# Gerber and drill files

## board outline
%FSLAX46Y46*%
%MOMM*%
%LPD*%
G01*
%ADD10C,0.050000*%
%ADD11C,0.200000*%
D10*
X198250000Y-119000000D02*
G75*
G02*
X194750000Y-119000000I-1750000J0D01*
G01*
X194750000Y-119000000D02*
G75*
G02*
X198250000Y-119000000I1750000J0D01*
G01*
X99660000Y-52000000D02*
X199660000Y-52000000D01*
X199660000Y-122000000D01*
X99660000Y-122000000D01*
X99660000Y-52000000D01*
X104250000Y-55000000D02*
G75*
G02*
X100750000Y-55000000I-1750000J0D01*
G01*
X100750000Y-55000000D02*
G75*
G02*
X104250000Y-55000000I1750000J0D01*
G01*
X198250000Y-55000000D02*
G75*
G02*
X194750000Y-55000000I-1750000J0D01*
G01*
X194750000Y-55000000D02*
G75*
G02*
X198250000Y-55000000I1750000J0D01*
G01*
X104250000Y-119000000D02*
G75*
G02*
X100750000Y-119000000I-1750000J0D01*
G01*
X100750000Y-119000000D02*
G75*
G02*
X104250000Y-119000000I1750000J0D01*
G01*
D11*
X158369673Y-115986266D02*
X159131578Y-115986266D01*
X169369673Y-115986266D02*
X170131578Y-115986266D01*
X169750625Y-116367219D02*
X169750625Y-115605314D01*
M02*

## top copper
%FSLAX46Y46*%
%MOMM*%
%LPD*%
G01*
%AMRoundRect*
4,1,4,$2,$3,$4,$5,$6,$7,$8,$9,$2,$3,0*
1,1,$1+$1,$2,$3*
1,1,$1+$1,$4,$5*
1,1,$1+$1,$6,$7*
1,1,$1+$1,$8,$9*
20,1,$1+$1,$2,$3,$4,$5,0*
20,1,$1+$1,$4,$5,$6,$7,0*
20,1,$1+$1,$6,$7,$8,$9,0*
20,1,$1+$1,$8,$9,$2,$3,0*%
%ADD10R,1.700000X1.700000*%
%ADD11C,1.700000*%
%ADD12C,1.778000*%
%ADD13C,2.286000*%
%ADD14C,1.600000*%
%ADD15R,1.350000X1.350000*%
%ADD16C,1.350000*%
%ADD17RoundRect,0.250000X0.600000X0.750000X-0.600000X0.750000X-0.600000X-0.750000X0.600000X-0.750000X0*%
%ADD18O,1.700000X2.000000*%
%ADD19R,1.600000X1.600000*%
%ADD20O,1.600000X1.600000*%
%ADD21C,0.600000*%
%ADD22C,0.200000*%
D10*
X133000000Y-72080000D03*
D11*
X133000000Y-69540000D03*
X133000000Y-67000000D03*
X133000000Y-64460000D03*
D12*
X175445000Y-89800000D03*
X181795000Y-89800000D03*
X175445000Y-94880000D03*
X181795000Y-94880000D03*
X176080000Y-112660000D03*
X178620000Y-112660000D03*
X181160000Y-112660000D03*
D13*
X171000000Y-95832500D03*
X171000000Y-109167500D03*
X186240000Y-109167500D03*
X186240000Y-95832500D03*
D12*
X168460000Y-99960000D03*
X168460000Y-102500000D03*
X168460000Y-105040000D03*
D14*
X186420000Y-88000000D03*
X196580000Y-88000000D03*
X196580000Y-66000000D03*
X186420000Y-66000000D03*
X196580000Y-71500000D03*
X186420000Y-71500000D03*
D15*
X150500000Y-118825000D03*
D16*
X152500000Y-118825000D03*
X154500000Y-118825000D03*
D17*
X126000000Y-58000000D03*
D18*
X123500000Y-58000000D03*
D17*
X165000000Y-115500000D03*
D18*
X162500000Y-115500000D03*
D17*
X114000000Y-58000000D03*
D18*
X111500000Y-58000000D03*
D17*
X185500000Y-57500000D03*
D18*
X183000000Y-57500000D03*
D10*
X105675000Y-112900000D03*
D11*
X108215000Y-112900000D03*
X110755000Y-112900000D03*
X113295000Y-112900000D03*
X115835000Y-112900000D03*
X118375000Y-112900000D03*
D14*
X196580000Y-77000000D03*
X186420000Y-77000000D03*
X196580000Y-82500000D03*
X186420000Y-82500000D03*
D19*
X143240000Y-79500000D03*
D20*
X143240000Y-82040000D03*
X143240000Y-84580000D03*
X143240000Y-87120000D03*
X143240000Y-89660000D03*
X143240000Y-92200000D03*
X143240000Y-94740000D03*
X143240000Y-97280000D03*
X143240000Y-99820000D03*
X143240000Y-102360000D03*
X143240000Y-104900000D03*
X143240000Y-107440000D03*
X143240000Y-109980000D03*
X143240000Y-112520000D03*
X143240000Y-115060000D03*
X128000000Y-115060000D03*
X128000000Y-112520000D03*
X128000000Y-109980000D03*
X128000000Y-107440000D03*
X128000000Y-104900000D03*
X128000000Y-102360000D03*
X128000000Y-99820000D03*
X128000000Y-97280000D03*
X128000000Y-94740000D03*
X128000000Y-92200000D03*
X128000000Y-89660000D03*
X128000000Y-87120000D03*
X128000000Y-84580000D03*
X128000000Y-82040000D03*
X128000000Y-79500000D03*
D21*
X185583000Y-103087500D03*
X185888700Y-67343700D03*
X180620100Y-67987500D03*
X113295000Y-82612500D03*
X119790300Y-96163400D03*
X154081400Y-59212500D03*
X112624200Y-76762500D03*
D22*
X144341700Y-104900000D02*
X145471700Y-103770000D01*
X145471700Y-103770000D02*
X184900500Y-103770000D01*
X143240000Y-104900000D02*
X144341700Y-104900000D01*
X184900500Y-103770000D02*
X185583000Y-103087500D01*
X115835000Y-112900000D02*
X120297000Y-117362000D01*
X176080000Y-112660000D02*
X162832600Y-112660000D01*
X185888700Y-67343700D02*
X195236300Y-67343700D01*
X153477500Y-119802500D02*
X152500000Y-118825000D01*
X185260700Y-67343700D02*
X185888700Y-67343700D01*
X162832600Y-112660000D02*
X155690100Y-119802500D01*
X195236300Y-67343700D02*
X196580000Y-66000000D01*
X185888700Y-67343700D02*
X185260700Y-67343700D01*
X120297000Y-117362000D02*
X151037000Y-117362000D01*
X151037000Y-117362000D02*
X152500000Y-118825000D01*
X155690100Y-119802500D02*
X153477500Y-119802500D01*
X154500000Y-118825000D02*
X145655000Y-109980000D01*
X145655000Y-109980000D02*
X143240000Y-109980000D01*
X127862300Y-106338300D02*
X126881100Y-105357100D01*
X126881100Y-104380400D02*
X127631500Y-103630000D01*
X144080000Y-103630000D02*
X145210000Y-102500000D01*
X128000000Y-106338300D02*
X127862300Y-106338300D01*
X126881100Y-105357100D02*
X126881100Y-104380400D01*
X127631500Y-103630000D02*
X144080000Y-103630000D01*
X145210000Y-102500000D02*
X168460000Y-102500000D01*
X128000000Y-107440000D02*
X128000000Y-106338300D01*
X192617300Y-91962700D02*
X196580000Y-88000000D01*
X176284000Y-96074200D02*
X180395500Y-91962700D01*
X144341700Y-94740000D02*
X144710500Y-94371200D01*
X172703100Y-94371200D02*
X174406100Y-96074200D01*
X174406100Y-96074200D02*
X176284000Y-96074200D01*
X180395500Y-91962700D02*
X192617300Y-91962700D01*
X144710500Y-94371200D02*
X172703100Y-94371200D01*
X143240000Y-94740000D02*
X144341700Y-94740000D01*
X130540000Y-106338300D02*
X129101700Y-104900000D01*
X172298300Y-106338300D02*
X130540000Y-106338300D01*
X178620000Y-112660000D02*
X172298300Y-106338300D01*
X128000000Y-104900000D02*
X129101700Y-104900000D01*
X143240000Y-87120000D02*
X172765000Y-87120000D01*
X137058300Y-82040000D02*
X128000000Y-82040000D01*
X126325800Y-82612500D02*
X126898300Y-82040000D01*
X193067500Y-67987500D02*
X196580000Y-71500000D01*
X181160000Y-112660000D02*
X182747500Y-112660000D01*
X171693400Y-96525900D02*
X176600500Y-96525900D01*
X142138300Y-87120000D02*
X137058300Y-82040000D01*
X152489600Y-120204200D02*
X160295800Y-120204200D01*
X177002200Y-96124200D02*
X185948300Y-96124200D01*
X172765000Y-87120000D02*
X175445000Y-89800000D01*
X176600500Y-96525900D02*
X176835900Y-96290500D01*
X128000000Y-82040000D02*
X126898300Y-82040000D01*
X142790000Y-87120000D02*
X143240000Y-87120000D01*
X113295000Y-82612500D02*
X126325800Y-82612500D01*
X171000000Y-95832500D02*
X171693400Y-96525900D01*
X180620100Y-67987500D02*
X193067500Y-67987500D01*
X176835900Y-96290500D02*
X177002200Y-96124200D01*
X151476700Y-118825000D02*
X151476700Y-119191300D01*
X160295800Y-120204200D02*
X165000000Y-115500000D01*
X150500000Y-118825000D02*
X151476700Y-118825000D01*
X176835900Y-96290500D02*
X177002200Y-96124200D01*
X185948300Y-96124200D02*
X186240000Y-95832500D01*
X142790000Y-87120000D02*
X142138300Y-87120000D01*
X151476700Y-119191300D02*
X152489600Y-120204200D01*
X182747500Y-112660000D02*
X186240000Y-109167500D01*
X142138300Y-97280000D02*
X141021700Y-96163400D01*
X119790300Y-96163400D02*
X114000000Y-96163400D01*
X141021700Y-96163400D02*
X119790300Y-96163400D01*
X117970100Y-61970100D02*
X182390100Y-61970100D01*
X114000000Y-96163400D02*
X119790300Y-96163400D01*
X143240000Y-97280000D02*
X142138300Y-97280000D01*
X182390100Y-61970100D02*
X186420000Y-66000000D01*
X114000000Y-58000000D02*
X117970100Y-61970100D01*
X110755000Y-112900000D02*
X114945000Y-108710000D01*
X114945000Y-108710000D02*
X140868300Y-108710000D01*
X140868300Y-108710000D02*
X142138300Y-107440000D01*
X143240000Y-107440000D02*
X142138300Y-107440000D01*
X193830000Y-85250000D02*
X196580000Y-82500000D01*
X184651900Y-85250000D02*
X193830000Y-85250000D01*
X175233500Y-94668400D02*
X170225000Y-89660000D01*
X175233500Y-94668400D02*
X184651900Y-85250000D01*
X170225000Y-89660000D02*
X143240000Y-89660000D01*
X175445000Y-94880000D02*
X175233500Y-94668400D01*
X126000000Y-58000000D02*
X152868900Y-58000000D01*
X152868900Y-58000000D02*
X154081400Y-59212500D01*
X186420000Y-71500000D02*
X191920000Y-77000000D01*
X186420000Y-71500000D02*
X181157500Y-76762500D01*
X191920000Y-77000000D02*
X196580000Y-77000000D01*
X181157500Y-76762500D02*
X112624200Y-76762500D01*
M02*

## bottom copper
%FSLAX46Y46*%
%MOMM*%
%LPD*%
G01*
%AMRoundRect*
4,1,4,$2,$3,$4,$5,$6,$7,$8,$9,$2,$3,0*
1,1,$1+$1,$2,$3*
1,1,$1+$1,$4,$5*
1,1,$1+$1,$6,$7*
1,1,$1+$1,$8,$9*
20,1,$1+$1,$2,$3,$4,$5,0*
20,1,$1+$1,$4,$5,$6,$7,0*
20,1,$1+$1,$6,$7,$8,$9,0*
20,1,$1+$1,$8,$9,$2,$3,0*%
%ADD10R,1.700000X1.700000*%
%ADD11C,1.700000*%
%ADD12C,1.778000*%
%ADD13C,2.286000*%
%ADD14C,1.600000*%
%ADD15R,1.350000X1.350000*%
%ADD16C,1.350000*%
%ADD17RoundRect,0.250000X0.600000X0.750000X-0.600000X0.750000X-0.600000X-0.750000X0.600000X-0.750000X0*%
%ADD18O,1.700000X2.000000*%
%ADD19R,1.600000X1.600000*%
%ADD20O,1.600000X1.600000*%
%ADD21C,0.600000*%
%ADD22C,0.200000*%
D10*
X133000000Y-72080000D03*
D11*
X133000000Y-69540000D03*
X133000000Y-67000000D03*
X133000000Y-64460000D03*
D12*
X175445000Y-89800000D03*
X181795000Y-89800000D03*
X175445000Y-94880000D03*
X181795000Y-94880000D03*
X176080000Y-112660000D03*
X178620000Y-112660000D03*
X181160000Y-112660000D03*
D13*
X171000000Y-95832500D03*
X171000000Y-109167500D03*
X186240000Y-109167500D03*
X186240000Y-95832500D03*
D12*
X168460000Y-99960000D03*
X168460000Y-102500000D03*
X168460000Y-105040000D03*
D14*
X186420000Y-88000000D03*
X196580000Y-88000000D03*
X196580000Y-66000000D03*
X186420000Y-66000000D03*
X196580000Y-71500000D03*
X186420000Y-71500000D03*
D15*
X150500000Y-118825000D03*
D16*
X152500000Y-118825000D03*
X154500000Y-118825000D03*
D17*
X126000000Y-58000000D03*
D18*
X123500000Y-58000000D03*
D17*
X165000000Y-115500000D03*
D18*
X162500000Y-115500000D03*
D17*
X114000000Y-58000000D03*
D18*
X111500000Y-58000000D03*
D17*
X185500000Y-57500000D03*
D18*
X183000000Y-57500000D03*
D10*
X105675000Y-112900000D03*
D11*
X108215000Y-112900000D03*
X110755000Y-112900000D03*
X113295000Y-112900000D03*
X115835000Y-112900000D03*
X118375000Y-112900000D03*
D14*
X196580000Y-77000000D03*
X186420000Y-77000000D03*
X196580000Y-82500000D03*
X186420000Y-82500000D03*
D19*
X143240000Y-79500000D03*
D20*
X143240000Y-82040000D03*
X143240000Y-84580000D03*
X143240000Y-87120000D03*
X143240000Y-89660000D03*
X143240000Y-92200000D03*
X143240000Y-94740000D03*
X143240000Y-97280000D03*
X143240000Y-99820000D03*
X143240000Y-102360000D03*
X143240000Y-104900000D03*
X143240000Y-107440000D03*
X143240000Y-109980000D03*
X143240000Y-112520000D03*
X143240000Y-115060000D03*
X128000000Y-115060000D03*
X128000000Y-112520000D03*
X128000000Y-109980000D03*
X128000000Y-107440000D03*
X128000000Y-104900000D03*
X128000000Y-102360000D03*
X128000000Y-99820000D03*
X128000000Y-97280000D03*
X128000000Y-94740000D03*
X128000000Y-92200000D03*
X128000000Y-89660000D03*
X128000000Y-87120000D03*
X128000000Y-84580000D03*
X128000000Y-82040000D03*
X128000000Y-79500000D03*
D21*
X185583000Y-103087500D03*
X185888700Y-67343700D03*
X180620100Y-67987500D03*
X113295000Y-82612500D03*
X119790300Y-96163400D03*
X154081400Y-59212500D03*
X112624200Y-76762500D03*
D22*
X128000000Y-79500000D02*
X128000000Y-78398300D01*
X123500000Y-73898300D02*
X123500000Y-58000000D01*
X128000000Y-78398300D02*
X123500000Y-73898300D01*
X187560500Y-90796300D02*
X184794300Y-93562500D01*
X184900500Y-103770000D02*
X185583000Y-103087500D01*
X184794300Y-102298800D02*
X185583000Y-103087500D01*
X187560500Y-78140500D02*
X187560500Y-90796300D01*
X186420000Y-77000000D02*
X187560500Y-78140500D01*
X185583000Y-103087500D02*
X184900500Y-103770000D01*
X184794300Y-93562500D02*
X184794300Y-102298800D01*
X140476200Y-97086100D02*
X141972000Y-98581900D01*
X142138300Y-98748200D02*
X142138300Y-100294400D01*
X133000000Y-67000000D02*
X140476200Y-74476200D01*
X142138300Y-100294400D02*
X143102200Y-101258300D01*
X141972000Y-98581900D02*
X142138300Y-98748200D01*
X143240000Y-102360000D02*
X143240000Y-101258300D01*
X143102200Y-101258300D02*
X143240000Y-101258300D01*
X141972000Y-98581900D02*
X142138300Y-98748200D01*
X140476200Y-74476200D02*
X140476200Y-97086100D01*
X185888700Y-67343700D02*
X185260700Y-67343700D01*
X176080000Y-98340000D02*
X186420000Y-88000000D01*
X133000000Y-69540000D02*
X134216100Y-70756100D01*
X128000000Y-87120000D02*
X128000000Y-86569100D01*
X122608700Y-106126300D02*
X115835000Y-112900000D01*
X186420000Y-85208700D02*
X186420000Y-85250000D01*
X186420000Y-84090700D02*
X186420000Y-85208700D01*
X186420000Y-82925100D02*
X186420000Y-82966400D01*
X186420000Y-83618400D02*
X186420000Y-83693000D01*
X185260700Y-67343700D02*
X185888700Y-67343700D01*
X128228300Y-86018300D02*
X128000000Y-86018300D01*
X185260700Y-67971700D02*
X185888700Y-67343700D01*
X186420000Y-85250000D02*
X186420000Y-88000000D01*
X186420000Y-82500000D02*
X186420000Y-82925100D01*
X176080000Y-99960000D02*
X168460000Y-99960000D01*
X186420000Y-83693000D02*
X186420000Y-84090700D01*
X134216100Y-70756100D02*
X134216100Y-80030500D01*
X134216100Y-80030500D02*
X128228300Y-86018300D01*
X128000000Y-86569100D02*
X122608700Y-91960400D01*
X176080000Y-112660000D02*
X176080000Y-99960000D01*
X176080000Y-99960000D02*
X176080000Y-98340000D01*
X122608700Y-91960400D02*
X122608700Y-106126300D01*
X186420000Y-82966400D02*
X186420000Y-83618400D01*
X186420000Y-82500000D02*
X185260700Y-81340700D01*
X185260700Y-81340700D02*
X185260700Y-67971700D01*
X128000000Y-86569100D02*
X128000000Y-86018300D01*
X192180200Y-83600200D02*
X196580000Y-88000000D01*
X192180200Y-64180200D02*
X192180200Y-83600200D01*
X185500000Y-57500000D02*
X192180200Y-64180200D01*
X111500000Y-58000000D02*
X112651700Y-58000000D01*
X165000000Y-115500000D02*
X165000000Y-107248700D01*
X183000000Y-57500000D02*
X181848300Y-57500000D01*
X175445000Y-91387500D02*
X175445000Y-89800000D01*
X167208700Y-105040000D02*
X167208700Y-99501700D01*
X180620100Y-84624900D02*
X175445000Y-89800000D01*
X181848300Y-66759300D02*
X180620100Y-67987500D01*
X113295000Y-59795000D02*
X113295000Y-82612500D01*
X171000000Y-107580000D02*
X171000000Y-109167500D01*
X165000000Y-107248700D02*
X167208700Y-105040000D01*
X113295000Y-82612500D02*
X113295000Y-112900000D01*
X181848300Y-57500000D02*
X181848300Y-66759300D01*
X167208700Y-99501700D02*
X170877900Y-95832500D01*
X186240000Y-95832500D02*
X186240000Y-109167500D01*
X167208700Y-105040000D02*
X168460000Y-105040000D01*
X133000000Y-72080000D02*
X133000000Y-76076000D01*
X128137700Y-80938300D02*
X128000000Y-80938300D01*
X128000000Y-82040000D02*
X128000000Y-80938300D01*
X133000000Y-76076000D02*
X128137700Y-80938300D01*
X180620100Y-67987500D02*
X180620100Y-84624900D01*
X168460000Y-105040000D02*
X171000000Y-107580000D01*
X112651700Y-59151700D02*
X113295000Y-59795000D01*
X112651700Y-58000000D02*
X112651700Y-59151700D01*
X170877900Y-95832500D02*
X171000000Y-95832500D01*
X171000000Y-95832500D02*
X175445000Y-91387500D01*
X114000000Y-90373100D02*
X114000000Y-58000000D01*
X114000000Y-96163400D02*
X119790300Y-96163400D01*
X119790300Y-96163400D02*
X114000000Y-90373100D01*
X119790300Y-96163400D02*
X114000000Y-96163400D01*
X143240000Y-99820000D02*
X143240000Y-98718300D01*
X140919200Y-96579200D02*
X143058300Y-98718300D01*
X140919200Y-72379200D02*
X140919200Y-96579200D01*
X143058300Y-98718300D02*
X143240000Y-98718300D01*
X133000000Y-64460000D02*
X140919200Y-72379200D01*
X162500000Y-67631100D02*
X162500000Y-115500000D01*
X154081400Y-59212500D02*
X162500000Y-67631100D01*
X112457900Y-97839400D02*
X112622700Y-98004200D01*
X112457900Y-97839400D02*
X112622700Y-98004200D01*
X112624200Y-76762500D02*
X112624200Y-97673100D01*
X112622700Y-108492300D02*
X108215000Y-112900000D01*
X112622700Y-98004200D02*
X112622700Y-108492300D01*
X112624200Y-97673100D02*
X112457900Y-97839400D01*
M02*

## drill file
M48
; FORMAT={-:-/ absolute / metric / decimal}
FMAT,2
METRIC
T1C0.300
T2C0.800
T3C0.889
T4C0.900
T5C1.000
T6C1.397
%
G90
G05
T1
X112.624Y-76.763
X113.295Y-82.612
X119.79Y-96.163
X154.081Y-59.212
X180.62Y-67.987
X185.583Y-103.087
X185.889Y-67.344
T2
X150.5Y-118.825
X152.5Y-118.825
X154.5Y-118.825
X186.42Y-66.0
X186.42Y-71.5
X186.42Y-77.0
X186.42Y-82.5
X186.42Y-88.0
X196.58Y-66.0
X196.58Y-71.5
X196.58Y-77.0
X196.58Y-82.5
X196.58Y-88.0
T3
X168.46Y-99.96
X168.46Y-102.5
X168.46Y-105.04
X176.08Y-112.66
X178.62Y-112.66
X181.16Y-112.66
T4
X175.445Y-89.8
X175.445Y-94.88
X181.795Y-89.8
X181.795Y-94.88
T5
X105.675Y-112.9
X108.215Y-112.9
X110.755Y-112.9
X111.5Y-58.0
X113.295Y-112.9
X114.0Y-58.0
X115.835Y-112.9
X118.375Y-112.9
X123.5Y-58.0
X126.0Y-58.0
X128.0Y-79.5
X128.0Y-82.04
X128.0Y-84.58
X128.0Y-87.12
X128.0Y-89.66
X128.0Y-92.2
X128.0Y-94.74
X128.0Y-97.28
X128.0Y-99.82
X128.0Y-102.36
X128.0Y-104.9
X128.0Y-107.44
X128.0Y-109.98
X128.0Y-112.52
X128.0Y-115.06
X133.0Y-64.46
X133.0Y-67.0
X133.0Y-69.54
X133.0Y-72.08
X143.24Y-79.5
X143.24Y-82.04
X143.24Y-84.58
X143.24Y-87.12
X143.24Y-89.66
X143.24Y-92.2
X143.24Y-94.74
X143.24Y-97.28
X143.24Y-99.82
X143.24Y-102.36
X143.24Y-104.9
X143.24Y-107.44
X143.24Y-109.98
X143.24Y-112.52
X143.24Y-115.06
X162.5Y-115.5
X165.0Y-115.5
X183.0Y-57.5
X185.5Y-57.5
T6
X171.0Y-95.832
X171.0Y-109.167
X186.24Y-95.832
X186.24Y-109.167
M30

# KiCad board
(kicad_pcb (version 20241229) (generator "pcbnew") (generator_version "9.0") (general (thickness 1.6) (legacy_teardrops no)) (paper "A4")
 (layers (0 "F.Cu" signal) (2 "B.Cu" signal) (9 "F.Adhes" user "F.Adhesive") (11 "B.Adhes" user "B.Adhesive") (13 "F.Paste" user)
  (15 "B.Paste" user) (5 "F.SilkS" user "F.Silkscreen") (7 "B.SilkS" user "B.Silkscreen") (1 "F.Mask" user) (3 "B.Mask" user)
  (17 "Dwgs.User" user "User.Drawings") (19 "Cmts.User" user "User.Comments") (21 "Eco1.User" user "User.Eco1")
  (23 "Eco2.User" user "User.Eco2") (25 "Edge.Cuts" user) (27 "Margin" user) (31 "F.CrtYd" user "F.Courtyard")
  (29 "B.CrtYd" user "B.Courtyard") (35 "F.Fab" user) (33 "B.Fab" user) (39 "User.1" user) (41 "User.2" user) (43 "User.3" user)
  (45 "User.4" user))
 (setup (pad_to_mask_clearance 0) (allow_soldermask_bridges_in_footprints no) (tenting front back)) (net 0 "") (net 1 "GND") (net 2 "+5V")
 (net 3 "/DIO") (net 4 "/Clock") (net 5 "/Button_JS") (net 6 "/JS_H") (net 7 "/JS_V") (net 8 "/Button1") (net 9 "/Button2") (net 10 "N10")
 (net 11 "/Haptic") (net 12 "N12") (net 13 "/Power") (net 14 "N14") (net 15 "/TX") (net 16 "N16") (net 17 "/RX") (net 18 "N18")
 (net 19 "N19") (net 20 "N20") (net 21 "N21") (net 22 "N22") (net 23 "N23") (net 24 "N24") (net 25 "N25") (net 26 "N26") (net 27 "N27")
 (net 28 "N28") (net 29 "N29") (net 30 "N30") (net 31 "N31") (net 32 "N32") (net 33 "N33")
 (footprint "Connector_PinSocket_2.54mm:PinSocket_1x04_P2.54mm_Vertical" (layer "F.Cu") (at 133 72.08 180)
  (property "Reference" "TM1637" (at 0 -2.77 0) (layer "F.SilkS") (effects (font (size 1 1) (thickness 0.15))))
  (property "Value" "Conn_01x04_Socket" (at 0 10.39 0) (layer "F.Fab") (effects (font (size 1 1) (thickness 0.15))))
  (pad "1" thru_hole rect (at 0 0 180) (size 1.7 1.7) (drill 1) (layers "*.Cu" "*.Mask") (remove_unused_layers no) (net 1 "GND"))
  (pad "2" thru_hole circle (at 0 2.54 180) (size 1.7 1.7) (drill 1) (layers "*.Cu" "*.Mask") (remove_unused_layers no) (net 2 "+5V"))
  (pad "3" thru_hole circle (at 0 5.08 180) (size 1.7 1.7) (drill 1) (layers "*.Cu" "*.Mask") (remove_unused_layers no) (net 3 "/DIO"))
  (pad "4" thru_hole circle (at 0 7.62 180) (size 1.7 1.7) (drill 1) (layers "*.Cu" "*.Mask") (remove_unused_layers no) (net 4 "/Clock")))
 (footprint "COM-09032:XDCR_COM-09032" (layer "F.Cu") (at 178.62 102.5)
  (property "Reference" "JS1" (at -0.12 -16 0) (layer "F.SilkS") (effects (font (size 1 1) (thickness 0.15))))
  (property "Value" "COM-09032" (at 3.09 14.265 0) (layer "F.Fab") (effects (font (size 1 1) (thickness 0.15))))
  (pad "B1A" thru_hole circle (at -3.175 -12.7) (size 1.778 1.778) (drill 0.9) (layers "*.Cu" "*.Mask") (remove_unused_layers no)
   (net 1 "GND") (solder_mask_margin 0.102))
  (pad "B1B" thru_hole circle (at 3.175 -12.7) (size 1.778 1.778) (drill 0.9) (layers "*.Cu" "*.Mask") (remove_unused_layers no)
   (solder_mask_margin 0.102))
  (pad "B2A" thru_hole circle (at -3.175 -7.62) (size 1.778 1.778) (drill 0.9) (layers "*.Cu" "*.Mask") (remove_unused_layers no)
   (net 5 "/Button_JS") (solder_mask_margin 0.102))
  (pad "B2B" thru_hole circle (at 3.175 -7.62) (size 1.778 1.778) (drill 0.9) (layers "*.Cu" "*.Mask") (remove_unused_layers no)
   (solder_mask_margin 0.102))
  (pad "H1" thru_hole circle (at -2.54 10.16) (size 1.778 1.778) (drill 0.889) (layers "*.Cu" "*.Mask") (remove_unused_layers no)
   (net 2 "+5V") (solder_mask_margin 0.102))
  (pad "H2" thru_hole circle (at 0 10.16) (size 1.778 1.778) (drill 0.889) (layers "*.Cu" "*.Mask") (remove_unused_layers no)
   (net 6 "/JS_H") (solder_mask_margin 0.102))
  (pad "H3" thru_hole circle (at 2.54 10.16) (size 1.778 1.778) (drill 0.889) (layers "*.Cu" "*.Mask") (remove_unused_layers no)
   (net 1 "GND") (solder_mask_margin 0.102))
  (pad "S1" thru_hole circle (at -7.62 -6.6675) (size 2.286 2.286) (drill 1.397) (layers "*.Cu" "*.Mask") (remove_unused_layers no)
   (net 1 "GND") (solder_mask_margin 0.102))
  (pad "S2" thru_hole circle (at -7.62 6.6675) (size 2.286 2.286) (drill 1.397) (layers "*.Cu" "*.Mask") (remove_unused_layers no)
   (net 1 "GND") (solder_mask_margin 0.102))
  (pad "S3" thru_hole circle (at 7.62 6.6675) (size 2.286 2.286) (drill 1.397) (layers "*.Cu" "*.Mask") (remove_unused_layers no)
   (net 1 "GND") (solder_mask_margin 0.102))
  (pad "S4" thru_hole circle (at 7.62 -6.6675) (size 2.286 2.286) (drill 1.397) (layers "*.Cu" "*.Mask") (remove_unused_layers no)
   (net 1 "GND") (solder_mask_margin 0.102))
  (pad "V1" thru_hole circle (at -10.16 -2.54) (size 1.778 1.778) (drill 0.889) (layers "*.Cu" "*.Mask") (remove_unused_layers no)
   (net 2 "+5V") (solder_mask_margin 0.102))
  (pad "V2" thru_hole circle (at -10.16 0) (size 1.778 1.778) (drill 0.889) (layers "*.Cu" "*.Mask") (remove_unused_layers no)
   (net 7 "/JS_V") (solder_mask_margin 0.102))
  (pad "V3" thru_hole circle (at -10.16 2.54) (size 1.778 1.778) (drill 0.889) (layers "*.Cu" "*.Mask") (remove_unused_layers no)
   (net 1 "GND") (solder_mask_margin 0.102)))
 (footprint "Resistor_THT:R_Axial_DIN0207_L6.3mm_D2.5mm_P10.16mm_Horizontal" (layer "B.Cu") (at 186.42 88)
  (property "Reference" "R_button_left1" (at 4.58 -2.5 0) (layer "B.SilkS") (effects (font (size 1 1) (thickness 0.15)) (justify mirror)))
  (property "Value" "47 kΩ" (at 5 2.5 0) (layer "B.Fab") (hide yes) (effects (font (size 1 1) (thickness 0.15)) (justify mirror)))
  (pad "1" thru_hole circle (at 0 0) (size 1.6 1.6) (drill 0.8) (layers "*.Cu" "*.Mask") (remove_unused_layers no) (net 2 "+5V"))
  (pad "2" thru_hole circle (at 10.16 0) (size 1.6 1.6) (drill 0.8) (layers "*.Cu" "*.Mask") (remove_unused_layers no) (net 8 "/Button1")))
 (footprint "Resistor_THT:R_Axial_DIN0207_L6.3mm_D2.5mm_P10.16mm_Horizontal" (layer "B.Cu") (at 196.58 66 180)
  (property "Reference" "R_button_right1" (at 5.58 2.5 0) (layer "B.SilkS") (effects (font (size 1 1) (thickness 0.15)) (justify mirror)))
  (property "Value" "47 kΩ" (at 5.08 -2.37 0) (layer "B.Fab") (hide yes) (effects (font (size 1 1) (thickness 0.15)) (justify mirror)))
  (pad "1" thru_hole circle (at 0 0 180) (size 1.6 1.6) (drill 0.8) (layers "*.Cu" "*.Mask") (remove_unused_layers no) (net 2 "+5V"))
  (pad "2" thru_hole circle (at 10.16 0 180) (size 1.6 1.6) (drill 0.8) (layers "*.Cu" "*.Mask") (remove_unused_layers no)
   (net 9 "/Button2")))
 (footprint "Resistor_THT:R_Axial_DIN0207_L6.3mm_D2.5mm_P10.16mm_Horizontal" (layer "B.Cu") (at 196.58 71.5 180)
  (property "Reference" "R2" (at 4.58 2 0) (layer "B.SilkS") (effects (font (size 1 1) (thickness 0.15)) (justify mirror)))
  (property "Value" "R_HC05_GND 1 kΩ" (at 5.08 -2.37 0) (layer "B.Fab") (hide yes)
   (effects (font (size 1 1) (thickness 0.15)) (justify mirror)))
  (pad "1" thru_hole circle (at 0 0 180) (size 1.6 1.6) (drill 0.8) (layers "*.Cu" "*.Mask") (remove_unused_layers no) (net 1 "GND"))
  (pad "2" thru_hole circle (at 10.16 0 180) (size 1.6 1.6) (drill 0.8) (layers "*.Cu" "*.Mask") (remove_unused_layers no) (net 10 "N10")))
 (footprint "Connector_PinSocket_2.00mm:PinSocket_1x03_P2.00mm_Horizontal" (layer "B.Cu") (at 150.5 118.825 -90)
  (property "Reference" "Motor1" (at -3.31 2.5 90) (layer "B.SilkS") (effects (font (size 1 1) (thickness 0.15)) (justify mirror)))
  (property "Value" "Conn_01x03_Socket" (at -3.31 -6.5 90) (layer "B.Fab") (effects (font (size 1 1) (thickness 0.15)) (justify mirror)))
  (pad "1" thru_hole rect (at 0 0 270) (size 1.35 1.35) (drill 0.8) (layers "*.Cu" "*.Mask") (remove_unused_layers no) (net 1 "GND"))
  (pad "2" thru_hole circle (at 0 -2 270) (size 1.35 1.35) (drill 0.8) (layers "*.Cu" "*.Mask") (remove_unused_layers no) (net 2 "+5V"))
  (pad "3" thru_hole circle (at 0 -4 270) (size 1.35 1.35) (drill 0.8) (layers "*.Cu" "*.Mask") (remove_unused_layers no) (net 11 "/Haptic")))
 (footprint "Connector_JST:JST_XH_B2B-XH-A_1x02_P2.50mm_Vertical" (layer "B.Cu") (at 126 58 180)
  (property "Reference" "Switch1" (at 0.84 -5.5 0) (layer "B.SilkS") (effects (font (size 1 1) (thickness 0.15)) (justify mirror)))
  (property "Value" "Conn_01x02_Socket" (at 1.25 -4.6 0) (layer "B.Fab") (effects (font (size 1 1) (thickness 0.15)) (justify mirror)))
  (pad "1" thru_hole roundrect (at 0 0 180) (size 1.7 2) (drill 1) (layers "*.Cu" "*.Mask") (remove_unused_layers no)
   (roundrect_rratio 0.147059) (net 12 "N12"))
  (pad "2" thru_hole oval (at 2.5 0 180) (size 1.7 2) (drill 1) (layers "*.Cu" "*.Mask") (remove_unused_layers no) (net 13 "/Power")))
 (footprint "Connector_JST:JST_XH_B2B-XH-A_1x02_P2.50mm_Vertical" (layer "B.Cu") (at 165 115.5 180)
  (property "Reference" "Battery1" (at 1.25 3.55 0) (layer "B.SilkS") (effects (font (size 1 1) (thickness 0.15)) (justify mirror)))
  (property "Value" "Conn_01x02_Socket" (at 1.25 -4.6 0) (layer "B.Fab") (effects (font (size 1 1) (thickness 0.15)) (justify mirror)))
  (pad "1" thru_hole roundrect (at 0 0 180) (size 1.7 2) (drill 1) (layers "*.Cu" "*.Mask") (remove_unused_layers no)
   (roundrect_rratio 0.147059) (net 1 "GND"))
  (pad "2" thru_hole oval (at 2.5 0 180) (size 1.7 2) (drill 1) (layers "*.Cu" "*.Mask") (remove_unused_layers no) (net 12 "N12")))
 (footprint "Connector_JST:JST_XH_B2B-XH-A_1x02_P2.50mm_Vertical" (layer "B.Cu") (at 114 58 180)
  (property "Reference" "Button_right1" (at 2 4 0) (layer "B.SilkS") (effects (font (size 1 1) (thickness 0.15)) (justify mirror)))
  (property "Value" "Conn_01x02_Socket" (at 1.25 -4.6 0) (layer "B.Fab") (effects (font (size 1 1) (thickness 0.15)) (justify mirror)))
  (pad "1" thru_hole roundrect (at 0 0 180) (size 1.7 2) (drill 1) (layers "*.Cu" "*.Mask") (remove_unused_layers no)
   (roundrect_rratio 0.147059) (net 9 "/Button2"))
  (pad "2" thru_hole oval (at 2.5 0 180) (size 1.7 2) (drill 1) (layers "*.Cu" "*.Mask") (remove_unused_layers no) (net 1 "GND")))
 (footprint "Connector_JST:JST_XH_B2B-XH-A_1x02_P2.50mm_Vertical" (layer "B.Cu") (at 185.5 57.5 180)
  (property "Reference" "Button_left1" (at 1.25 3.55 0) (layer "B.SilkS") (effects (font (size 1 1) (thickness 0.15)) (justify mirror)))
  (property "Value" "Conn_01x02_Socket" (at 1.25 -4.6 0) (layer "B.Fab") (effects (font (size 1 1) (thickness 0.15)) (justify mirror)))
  (pad "1" thru_hole roundrect (at 0 0 180) (size 1.7 2) (drill 1) (layers "*.Cu" "*.Mask") (remove_unused_layers no)
   (roundrect_rratio 0.147059) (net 8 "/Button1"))
  (pad "2" thru_hole oval (at 2.5 0 180) (size 1.7 2) (drill 1) (layers "*.Cu" "*.Mask") (remove_unused_layers no) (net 1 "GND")))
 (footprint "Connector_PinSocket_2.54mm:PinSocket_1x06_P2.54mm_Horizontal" (layer "B.Cu") (at 105.675 112.9 -90)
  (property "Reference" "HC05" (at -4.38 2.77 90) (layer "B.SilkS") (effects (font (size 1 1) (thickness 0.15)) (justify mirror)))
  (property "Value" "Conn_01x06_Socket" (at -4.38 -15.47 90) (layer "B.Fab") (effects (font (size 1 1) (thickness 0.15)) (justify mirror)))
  (pad "1" thru_hole rect (at 0 0 270) (size 1.7 1.7) (drill 1) (layers "*.Cu" "*.Mask") (remove_unused_layers no) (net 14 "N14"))
  (pad "2" thru_hole circle (at 0 -2.54 270) (size 1.7 1.7) (drill 1) (layers "*.Cu" "*.Mask") (remove_unused_layers no) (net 10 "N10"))
  (pad "3" thru_hole circle (at 0 -5.08 270) (size 1.7 1.7) (drill 1) (layers "*.Cu" "*.Mask") (remove_unused_layers no) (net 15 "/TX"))
  (pad "4" thru_hole circle (at 0 -7.62 270) (size 1.7 1.7) (drill 1) (layers "*.Cu" "*.Mask") (remove_unused_layers no) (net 1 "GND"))
  (pad "5" thru_hole circle (at 0 -10.16 270) (size 1.7 1.7) (drill 1) (layers "*.Cu" "*.Mask") (remove_unused_layers no) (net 2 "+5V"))
  (pad "6" thru_hole circle (at 0 -12.7 270) (size 1.7 1.7) (drill 1) (layers "*.Cu" "*.Mask") (remove_unused_layers no) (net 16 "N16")))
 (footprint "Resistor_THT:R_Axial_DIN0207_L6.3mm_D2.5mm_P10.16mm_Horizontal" (layer "B.Cu") (at 196.58 77 180)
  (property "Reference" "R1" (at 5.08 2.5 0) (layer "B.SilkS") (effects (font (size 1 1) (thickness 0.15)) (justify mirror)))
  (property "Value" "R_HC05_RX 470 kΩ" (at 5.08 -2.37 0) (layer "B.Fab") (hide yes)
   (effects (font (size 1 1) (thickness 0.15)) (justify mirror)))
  (pad "1" thru_hole circle (at 0 0 180) (size 1.6 1.6) (drill 0.8) (layers "*.Cu" "*.Mask") (remove_unused_layers no) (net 10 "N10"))
  (pad "2" thru_hole circle (at 10.16 0 180) (size 1.6 1.6) (drill 0.8) (layers "*.Cu" "*.Mask") (remove_unused_layers no) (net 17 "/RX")))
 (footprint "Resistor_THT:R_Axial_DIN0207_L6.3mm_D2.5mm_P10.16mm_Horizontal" (layer "B.Cu") (at 196.58 82.5 180)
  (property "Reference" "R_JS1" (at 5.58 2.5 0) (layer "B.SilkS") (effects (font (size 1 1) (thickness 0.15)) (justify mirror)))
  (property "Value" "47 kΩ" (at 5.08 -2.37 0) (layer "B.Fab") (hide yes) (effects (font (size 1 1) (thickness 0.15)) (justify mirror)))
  (pad "1" thru_hole circle (at 0 0 180) (size 1.6 1.6) (drill 0.8) (layers "*.Cu" "*.Mask") (remove_unused_layers no) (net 5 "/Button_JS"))
  (pad "2" thru_hole circle (at 10.16 0 180) (size 1.6 1.6) (drill 0.8) (layers "*.Cu" "*.Mask") (remove_unused_layers no) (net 2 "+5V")))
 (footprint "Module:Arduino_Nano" (layer "B.Cu") (at 143.24 79.5 180)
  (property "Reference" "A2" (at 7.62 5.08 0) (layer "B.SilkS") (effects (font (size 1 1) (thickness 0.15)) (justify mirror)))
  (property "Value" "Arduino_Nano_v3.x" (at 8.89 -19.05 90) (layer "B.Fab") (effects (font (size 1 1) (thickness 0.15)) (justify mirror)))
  (pad "1" thru_hole rect (at 0 0 180) (size 1.6 1.6) (drill 1) (layers "*.Cu" "*.Mask") (remove_unused_layers no) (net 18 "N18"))
  (pad "2" thru_hole oval (at 0 -2.54 180) (size 1.6 1.6) (drill 1) (layers "*.Cu" "*.Mask") (remove_unused_layers no) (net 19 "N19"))
  (pad "3" thru_hole oval (at 0 -5.08 180) (size 1.6 1.6) (drill 1) (layers "*.Cu" "*.Mask") (remove_unused_layers no) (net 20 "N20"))
  (pad "4" thru_hole oval (at 0 -7.62 180) (size 1.6 1.6) (drill 1) (layers "*.Cu" "*.Mask") (remove_unused_layers no) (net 1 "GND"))
  (pad "5" thru_hole oval (at 0 -10.16 180) (size 1.6 1.6) (drill 1) (layers "*.Cu" "*.Mask") (remove_unused_layers no) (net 5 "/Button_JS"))
  (pad "6" thru_hole oval (at 0 -12.7 180) (size 1.6 1.6) (drill 1) (layers "*.Cu" "*.Mask") (remove_unused_layers no) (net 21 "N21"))
  (pad "7" thru_hole oval (at 0 -15.24 180) (size 1.6 1.6) (drill 1) (layers "*.Cu" "*.Mask") (remove_unused_layers no) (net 8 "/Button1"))
  (pad "8" thru_hole oval (at 0 -17.78 180) (size 1.6 1.6) (drill 1) (layers "*.Cu" "*.Mask") (remove_unused_layers no) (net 9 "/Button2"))
  (pad "9" thru_hole oval (at 0 -20.32 180) (size 1.6 1.6) (drill 1) (layers "*.Cu" "*.Mask") (remove_unused_layers no) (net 4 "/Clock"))
  (pad "10" thru_hole oval (at 0 -22.86 180) (size 1.6 1.6) (drill 1) (layers "*.Cu" "*.Mask") (remove_unused_layers no) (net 3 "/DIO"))
  (pad "11" thru_hole oval (at 0 -25.4 180) (size 1.6 1.6) (drill 1) (layers "*.Cu" "*.Mask") (remove_unused_layers no) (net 17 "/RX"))
  (pad "12" thru_hole oval (at 0 -27.94 180) (size 1.6 1.6) (drill 1) (layers "*.Cu" "*.Mask") (remove_unused_layers no) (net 15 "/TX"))
  (pad "13" thru_hole oval (at 0 -30.48 180) (size 1.6 1.6) (drill 1) (layers "*.Cu" "*.Mask") (remove_unused_layers no) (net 11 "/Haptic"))
  (pad "14" thru_hole oval (at 0 -33.02 180) (size 1.6 1.6) (drill 1) (layers "*.Cu" "*.Mask") (remove_unused_layers no) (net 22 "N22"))
  (pad "15" thru_hole oval (at 0 -35.56 180) (size 1.6 1.6) (drill 1) (layers "*.Cu" "*.Mask") (remove_unused_layers no) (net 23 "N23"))
  (pad "16" thru_hole oval (at 15.24 -35.56 180) (size 1.6 1.6) (drill 1) (layers "*.Cu" "*.Mask") (remove_unused_layers no) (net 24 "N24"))
  (pad "17" thru_hole oval (at 15.24 -33.02 180) (size 1.6 1.6) (drill 1) (layers "*.Cu" "*.Mask") (remove_unused_layers no) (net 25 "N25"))
  (pad "18" thru_hole oval (at 15.24 -30.48 180) (size 1.6 1.6) (drill 1) (layers "*.Cu" "*.Mask") (remove_unused_layers no) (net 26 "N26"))
  (pad "19" thru_hole oval (at 15.24 -27.94 180) (size 1.6 1.6) (drill 1) (layers "*.Cu" "*.Mask") (remove_unused_layers no) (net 7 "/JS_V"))
  (pad "20" thru_hole oval (at 15.24 -25.4 180) (size 1.6 1.6) (drill 1) (layers "*.Cu" "*.Mask") (remove_unused_layers no) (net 6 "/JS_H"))
  (pad "21" thru_hole oval (at 15.24 -22.86 180) (size 1.6 1.6) (drill 1) (layers "*.Cu" "*.Mask") (remove_unused_layers no) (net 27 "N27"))
  (pad "22" thru_hole oval (at 15.24 -20.32 180) (size 1.6 1.6) (drill 1) (layers "*.Cu" "*.Mask") (remove_unused_layers no) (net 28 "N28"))
  (pad "23" thru_hole oval (at 15.24 -17.78 180) (size 1.6 1.6) (drill 1) (layers "*.Cu" "*.Mask") (remove_unused_layers no) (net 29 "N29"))
  (pad "24" thru_hole oval (at 15.24 -15.24 180) (size 1.6 1.6) (drill 1) (layers "*.Cu" "*.Mask") (remove_unused_layers no) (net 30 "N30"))
  (pad "25" thru_hole oval (at 15.24 -12.7 180) (size 1.6 1.6) (drill 1) (layers "*.Cu" "*.Mask") (remove_unused_layers no) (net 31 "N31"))
  (pad "26" thru_hole oval (at 15.24 -10.16 180) (size 1.6 1.6) (drill 1) (layers "*.Cu" "*.Mask") (remove_unused_layers no) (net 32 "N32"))
  (pad "27" thru_hole oval (at 15.24 -7.62 180) (size 1.6 1.6) (drill 1) (layers "*.Cu" "*.Mask") (remove_unused_layers no) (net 2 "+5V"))
  (pad "28" thru_hole oval (at 15.24 -5.08 180) (size 1.6 1.6) (drill 1) (layers "*.Cu" "*.Mask") (remove_unused_layers no) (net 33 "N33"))
  (pad "29" thru_hole oval (at 15.24 -2.54 180) (size 1.6 1.6) (drill 1) (layers "*.Cu" "*.Mask") (remove_unused_layers no) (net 1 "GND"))
  (pad "30" thru_hole oval (at 15.24 0 180) (size 1.6 1.6) (drill 1) (layers "*.Cu" "*.Mask") (remove_unused_layers no) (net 13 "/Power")))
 (gr_circle (center 196.5 119) (end 198.25 119) (stroke (width 0.05) (type solid)) (fill no) (layer "Edge.Cuts"))
 (gr_rect (start 99.66 52) (end 199.66 122) (stroke (width 0.05) (type default)) (fill no) (layer "Edge.Cuts"))
 (gr_circle (center 102.5 55) (end 104.25 55) (stroke (width 0.05) (type solid)) (fill no) (layer "Edge.Cuts"))
 (gr_circle (center 196.5 55) (end 198.25 55) (stroke (width 0.05) (type solid)) (fill no) (layer "Edge.Cuts"))
 (gr_circle (center 102.5 119) (end 104.25 119) (stroke (width 0.05) (type solid)) (fill no) (layer "Edge.Cuts"))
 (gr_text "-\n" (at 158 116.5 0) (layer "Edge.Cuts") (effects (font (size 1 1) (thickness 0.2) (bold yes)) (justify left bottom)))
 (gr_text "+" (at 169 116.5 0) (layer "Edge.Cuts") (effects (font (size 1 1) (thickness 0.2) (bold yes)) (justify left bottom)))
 (segment (start 128 79.5) (end 128 78.3983) (width 0.2) (layer "B.Cu") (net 13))
 (segment (start 123.5 73.8983) (end 123.5 58) (width 0.2) (layer "B.Cu") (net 13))
 (segment (start 128 78.3983) (end 123.5 73.8983) (width 0.2) (layer "B.Cu") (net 13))
 (segment (start 144.3417 104.9) (end 145.4717 103.77) (width 0.2) (layer "F.Cu") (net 17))
 (segment (start 145.4717 103.77) (end 184.9005 103.77) (width 0.2) (layer "F.Cu") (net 17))
 (segment (start 143.24 104.9) (end 144.3417 104.9) (width 0.2) (layer "F.Cu") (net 17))
 (segment (start 184.9005 103.77) (end 185.583 103.0875) (width 0.2) (layer "F.Cu") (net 17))
 (via (at 185.583 103.0875) (size 0.6) (drill 0.3) (layers "F.Cu" "B.Cu") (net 17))
 (segment (start 187.5605 90.7963) (end 184.7943 93.5625) (width 0.2) (layer "B.Cu") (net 17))
 (segment (start 184.9005 103.77) (end 185.583 103.0875) (width 0.2) (layer "B.Cu") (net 17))
 (segment (start 184.7943 102.2988) (end 185.583 103.0875) (width 0.2) (layer "B.Cu") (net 17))
 (segment (start 187.5605 78.1405) (end 187.5605 90.7963) (width 0.2) (layer "B.Cu") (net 17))
 (segment (start 186.42 77) (end 187.5605 78.1405) (width 0.2) (layer "B.Cu") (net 17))
 (segment (start 185.583 103.0875) (end 184.9005 103.77) (width 0.2) (layer "B.Cu") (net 17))
 (segment (start 184.7943 93.5625) (end 184.7943 102.2988) (width 0.2) (layer "B.Cu") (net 17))
 (segment (start 140.4762 97.0861) (end 141.972 98.5819) (width 0.2) (layer "B.Cu") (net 3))
 (segment (start 142.1383 98.7482) (end 142.1383 100.2944) (width 0.2) (layer "B.Cu") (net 3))
 (segment (start 133 67) (end 140.4762 74.4762) (width 0.2) (layer "B.Cu") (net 3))
 (segment (start 142.1383 100.2944) (end 143.1022 101.2583) (width 0.2) (layer "B.Cu") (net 3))
 (segment (start 141.972 98.5819) (end 142.1383 98.7482) (width 0.2) (layer "B.Cu") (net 3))
 (segment (start 143.24 102.36) (end 143.24 101.2583) (width 0.2) (layer "B.Cu") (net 3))
 (segment (start 143.1022 101.2583) (end 143.24 101.2583) (width 0.2) (layer "B.Cu") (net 3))
 (segment (start 141.972 98.5819) (end 142.1383 98.7482) (width 0.2) (layer "B.Cu") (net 3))
 (segment (start 140.4762 74.4762) (end 140.4762 97.0861) (width 0.2) (layer "B.Cu") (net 3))
 (segment (start 115.835 112.9) (end 120.297 117.362) (width 0.2) (layer "F.Cu") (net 2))
 (segment (start 176.08 112.66) (end 162.8326 112.66) (width 0.2) (layer "F.Cu") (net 2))
 (segment (start 185.8887 67.3437) (end 195.2363 67.3437) (width 0.2) (layer "F.Cu") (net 2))
 (segment (start 153.4775 119.8025) (end 152.5 118.825) (width 0.2) (layer "F.Cu") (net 2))
 (segment (start 185.2607 67.3437) (end 185.8887 67.3437) (width 0.2) (layer "F.Cu") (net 2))
 (segment (start 162.8326 112.66) (end 155.6901 119.8025) (width 0.2) (layer "F.Cu") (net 2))
 (segment (start 195.2363 67.3437) (end 196.58 66) (width 0.2) (layer "F.Cu") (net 2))
 (segment (start 185.8887 67.3437) (end 185.2607 67.3437) (width 0.2) (layer "F.Cu") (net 2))
 (segment (start 120.297 117.362) (end 151.037 117.362) (width 0.2) (layer "F.Cu") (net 2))
 (segment (start 151.037 117.362) (end 152.5 118.825) (width 0.2) (layer "F.Cu") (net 2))
 (segment (start 155.6901 119.8025) (end 153.4775 119.8025) (width 0.2) (layer "F.Cu") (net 2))
 (via (at 185.8887 67.3437) (size 0.6) (drill 0.3) (layers "F.Cu" "B.Cu") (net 2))
 (segment (start 185.8887 67.3437) (end 185.2607 67.3437) (width 0.2) (layer "B.Cu") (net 2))
 (segment (start 176.08 98.34) (end 186.42 88) (width 0.2) (layer "B.Cu") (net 2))
 (segment (start 133 69.54) (end 134.2161 70.7561) (width 0.2) (layer "B.Cu") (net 2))
 (segment (start 128 87.12) (end 128 86.5691) (width 0.2) (layer "B.Cu") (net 2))
 (segment (start 122.6087 106.1263) (end 115.835 112.9) (width 0.2) (layer "B.Cu") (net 2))
 (segment (start 186.42 85.2087) (end 186.42 85.25) (width 0.2) (layer "B.Cu") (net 2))
 (segment (start 186.42 84.0907) (end 186.42 85.2087) (width 0.2) (layer "B.Cu") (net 2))
 (segment (start 186.42 82.9251) (end 186.42 82.9664) (width 0.2) (layer "B.Cu") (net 2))
 (segment (start 186.42 83.6184) (end 186.42 83.693) (width 0.2) (layer "B.Cu") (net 2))
 (segment (start 185.2607 67.3437) (end 185.8887 67.3437) (width 0.2) (layer "B.Cu") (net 2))
 (segment (start 128.2283 86.0183) (end 128 86.0183) (width 0.2) (layer "B.Cu") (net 2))
 (segment (start 185.2607 67.9717) (end 185.8887 67.3437) (width 0.2) (layer "B.Cu") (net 2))
 (segment (start 186.42 85.25) (end 186.42 88) (width 0.2) (layer "B.Cu") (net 2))
 (segment (start 186.42 82.5) (end 186.42 82.9251) (width 0.2) (layer "B.Cu") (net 2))
 (segment (start 176.08 99.96) (end 168.46 99.96) (width 0.2) (layer "B.Cu") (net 2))
 (segment (start 186.42 83.693) (end 186.42 84.0907) (width 0.2) (layer "B.Cu") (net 2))
 (segment (start 134.2161 70.7561) (end 134.2161 80.0305) (width 0.2) (layer "B.Cu") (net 2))
 (segment (start 134.2161 80.0305) (end 128.2283 86.0183) (width 0.2) (layer "B.Cu") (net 2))
 (segment (start 128 86.5691) (end 122.6087 91.9604) (width 0.2) (layer "B.Cu") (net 2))
 (segment (start 176.08 112.66) (end 176.08 99.96) (width 0.2) (layer "B.Cu") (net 2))
 (segment (start 176.08 99.96) (end 176.08 98.34) (width 0.2) (layer "B.Cu") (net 2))
 (segment (start 122.6087 91.9604) (end 122.6087 106.1263) (width 0.2) (layer "B.Cu") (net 2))
 (segment (start 186.42 82.9664) (end 186.42 83.6184) (width 0.2) (layer "B.Cu") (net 2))
 (segment (start 186.42 82.5) (end 185.2607 81.3407) (width 0.2) (layer "B.Cu") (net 2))
 (segment (start 185.2607 81.3407) (end 185.2607 67.9717) (width 0.2) (layer "B.Cu") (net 2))
 (segment (start 128 86.5691) (end 128 86.0183) (width 0.2) (layer "B.Cu") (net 2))
 (segment (start 154.5 118.825) (end 145.655 109.98) (width 0.2) (layer "F.Cu") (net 11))
 (segment (start 145.655 109.98) (end 143.24 109.98) (width 0.2) (layer "F.Cu") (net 11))
 (segment (start 127.8623 106.3383) (end 126.8811 105.3571) (width 0.2) (layer "F.Cu") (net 7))
 (segment (start 126.8811 104.3804) (end 127.6315 103.63) (width 0.2) (layer "F.Cu") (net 7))
 (segment (start 144.08 103.63) (end 145.21 102.5) (width 0.2) (layer "F.Cu") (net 7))
 (segment (start 128 106.3383) (end 127.8623 106.3383) (width 0.2) (layer "F.Cu") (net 7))
 (segment (start 126.8811 105.3571) (end 126.8811 104.3804) (width 0.2) (layer "F.Cu") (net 7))
 (segment (start 127.6315 103.63) (end 144.08 103.63) (width 0.2) (layer "F.Cu") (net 7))
 (segment (start 145.21 102.5) (end 168.46 102.5) (width 0.2) (layer "F.Cu") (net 7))
 (segment (start 128 107.44) (end 128 106.3383) (width 0.2) (layer "F.Cu") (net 7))
 (segment (start 192.6173 91.9627) (end 196.58 88) (width 0.2) (layer "F.Cu") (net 8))
 (segment (start 176.284 96.0742) (end 180.3955 91.9627) (width 0.2) (layer "F.Cu") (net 8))
 (segment (start 144.3417 94.74) (end 144.7105 94.3712) (width 0.2) (layer "F.Cu") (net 8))
 (segment (start 172.7031 94.3712) (end 174.4061 96.0742) (width 0.2) (layer "F.Cu") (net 8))
 (segment (start 174.4061 96.0742) (end 176.284 96.0742) (width 0.2) (layer "F.Cu") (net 8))
 (segment (start 180.3955 91.9627) (end 192.6173 91.9627) (width 0.2) (layer "F.Cu") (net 8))
 (segment (start 144.7105 94.3712) (end 172.7031 94.3712) (width 0.2) (layer "F.Cu") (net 8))
 (segment (start 143.24 94.74) (end 144.3417 94.74) (width 0.2) (layer "F.Cu") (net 8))
 (segment (start 192.1802 83.6002) (end 196.58 88) (width 0.2) (layer "B.Cu") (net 8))
 (segment (start 192.1802 64.1802) (end 192.1802 83.6002) (width 0.2) (layer "B.Cu") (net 8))
 (segment (start 185.5 57.5) (end 192.1802 64.1802) (width 0.2) (layer "B.Cu") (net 8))
 (segment (start 130.54 106.3383) (end 129.1017 104.9) (width 0.2) (layer "F.Cu") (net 6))
 (segment (start 172.2983 106.3383) (end 130.54 106.3383) (width 0.2) (layer "F.Cu") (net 6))
 (segment (start 178.62 112.66) (end 172.2983 106.3383) (width 0.2) (layer "F.Cu") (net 6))
 (segment (start 128 104.9) (end 129.1017 104.9) (width 0.2) (layer "F.Cu") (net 6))
 (segment (start 143.24 87.12) (end 172.765 87.12) (width 0.2) (layer "F.Cu") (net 1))
 (segment (start 137.0583 82.04) (end 128 82.04) (width 0.2) (layer "F.Cu") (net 1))
 (segment (start 126.3258 82.6125) (end 126.8983 82.04) (width 0.2) (layer "F.Cu") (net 1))
 (segment (start 193.0675 67.9875) (end 196.58 71.5) (width 0.2) (layer "F.Cu") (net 1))
 (segment (start 181.16 112.66) (end 182.7475 112.66) (width 0.2) (layer "F.Cu") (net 1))
 (segment (start 171.6934 96.5259) (end 176.6005 96.5259) (width 0.2) (layer "F.Cu") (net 1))
 (segment (start 142.1383 87.12) (end 137.0583 82.04) (width 0.2) (layer "F.Cu") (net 1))
 (segment (start 152.4896 120.2042) (end 160.2958 120.2042) (width 0.2) (layer "F.Cu") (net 1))
 (segment (start 177.0022 96.1242) (end 185.9483 96.1242) (width 0.2) (layer "F.Cu") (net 1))
 (segment (start 172.765 87.12) (end 175.445 89.8) (width 0.2) (layer "F.Cu") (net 1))
 (segment (start 176.6005 96.5259) (end 176.8359 96.2905) (width 0.2) (layer "F.Cu") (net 1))
 (segment (start 128 82.04) (end 126.8983 82.04) (width 0.2) (layer "F.Cu") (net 1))
 (segment (start 142.79 87.12) (end 143.24 87.12) (width 0.2) (layer "F.Cu") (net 1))
 (segment (start 113.295 82.6125) (end 126.3258 82.6125) (width 0.2) (layer "F.Cu") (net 1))
 (segment (start 171 95.8325) (end 171.6934 96.5259) (width 0.2) (layer "F.Cu") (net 1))
 (segment (start 180.6201 67.9875) (end 193.0675 67.9875) (width 0.2) (layer "F.Cu") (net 1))
 (segment (start 176.8359 96.2905) (end 177.0022 96.1242) (width 0.2) (layer "F.Cu") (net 1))
 (segment (start 151.4767 118.825) (end 151.4767 119.1913) (width 0.2) (layer "F.Cu") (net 1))
 (segment (start 160.2958 120.2042) (end 165 115.5) (width 0.2) (layer "F.Cu") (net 1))
 (segment (start 150.5 118.825) (end 151.4767 118.825) (width 0.2) (layer "F.Cu") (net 1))
 (segment (start 176.8359 96.2905) (end 177.0022 96.1242) (width 0.2) (layer "F.Cu") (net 1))
 (segment (start 185.9483 96.1242) (end 186.24 95.8325) (width 0.2) (layer "F.Cu") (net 1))
 (segment (start 142.79 87.12) (end 142.1383 87.12) (width 0.2) (layer "F.Cu") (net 1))
 (segment (start 151.4767 119.1913) (end 152.4896 120.2042) (width 0.2) (layer "F.Cu") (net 1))
 (segment (start 182.7475 112.66) (end 186.24 109.1675) (width 0.2) (layer "F.Cu") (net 1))
 (via (at 180.6201 67.9875) (size 0.6) (drill 0.3) (layers "F.Cu" "B.Cu") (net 1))
 (via (at 113.295 82.6125) (size 0.6) (drill 0.3) (layers "F.Cu" "B.Cu") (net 1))
 (segment (start 111.5 58) (end 112.6517 58) (width 0.2) (layer "B.Cu") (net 1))
 (segment (start 165 115.5) (end 165 107.2487) (width 0.2) (layer "B.Cu") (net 1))
 (segment (start 183 57.5) (end 181.8483 57.5) (width 0.2) (layer "B.Cu") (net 1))
 (segment (start 175.445 91.3875) (end 175.445 89.8) (width 0.2) (layer "B.Cu") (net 1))
 (segment (start 167.2087 105.04) (end 167.2087 99.5017) (width 0.2) (layer "B.Cu") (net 1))
 (segment (start 180.6201 84.6249) (end 175.445 89.8) (width 0.2) (layer "B.Cu") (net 1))
 (segment (start 181.8483 66.7593) (end 180.6201 67.9875) (width 0.2) (layer "B.Cu") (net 1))
 (segment (start 113.295 59.795) (end 113.295 82.6125) (width 0.2) (layer "B.Cu") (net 1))
 (segment (start 171 107.58) (end 171 109.1675) (width 0.2) (layer "B.Cu") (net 1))
 (segment (start 165 107.2487) (end 167.2087 105.04) (width 0.2) (layer "B.Cu") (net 1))
 (segment (start 113.295 82.6125) (end 113.295 112.9) (width 0.2) (layer "B.Cu") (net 1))
 (segment (start 181.8483 57.5) (end 181.8483 66.7593) (width 0.2) (layer "B.Cu") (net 1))
 (segment (start 167.2087 99.5017) (end 170.8779 95.8325) (width 0.2) (layer "B.Cu") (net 1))
 (segment (start 186.24 95.8325) (end 186.24 109.1675) (width 0.2) (layer "B.Cu") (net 1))
 (segment (start 167.2087 105.04) (end 168.46 105.04) (width 0.2) (layer "B.Cu") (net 1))
 (segment (start 133 72.08) (end 133 76.076) (width 0.2) (layer "B.Cu") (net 1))
 (segment (start 128.1377 80.9383) (end 128 80.9383) (width 0.2) (layer "B.Cu") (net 1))
 (segment (start 128 82.04) (end 128 80.9383) (width 0.2) (layer "B.Cu") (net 1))
 (segment (start 133 76.076) (end 128.1377 80.9383) (width 0.2) (layer "B.Cu") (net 1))
 (segment (start 180.6201 67.9875) (end 180.6201 84.6249) (width 0.2) (layer "B.Cu") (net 1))
 (segment (start 168.46 105.04) (end 171 107.58) (width 0.2) (layer "B.Cu") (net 1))
 (segment (start 112.6517 59.1517) (end 113.295 59.795) (width 0.2) (layer "B.Cu") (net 1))
 (segment (start 112.6517 58) (end 112.6517 59.1517) (width 0.2) (layer "B.Cu") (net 1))
 (segment (start 170.8779 95.8325) (end 171 95.8325) (width 0.2) (layer "B.Cu") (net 1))
 (segment (start 171 95.8325) (end 175.445 91.3875) (width 0.2) (layer "B.Cu") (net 1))
 (segment (start 142.1383 97.28) (end 141.0217 96.1634) (width 0.2) (layer "F.Cu") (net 9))
 (segment (start 119.7903 96.1634) (end 114 96.1634) (width 0.2) (layer "F.Cu") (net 9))
 (segment (start 141.0217 96.1634) (end 119.7903 96.1634) (width 0.2) (layer "F.Cu") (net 9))
 (segment (start 117.9701 61.9701) (end 182.3901 61.9701) (width 0.2) (layer "F.Cu") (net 9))
 (segment (start 114 96.1634) (end 119.7903 96.1634) (width 0.2) (layer "F.Cu") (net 9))
 (segment (start 143.24 97.28) (end 142.1383 97.28) (width 0.2) (layer "F.Cu") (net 9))
 (segment (start 182.3901 61.9701) (end 186.42 66) (width 0.2) (layer "F.Cu") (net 9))
 (segment (start 114 58) (end 117.9701 61.9701) (width 0.2) (layer "F.Cu") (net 9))
 (via (at 119.7903 96.1634) (size 0.6) (drill 0.3) (layers "F.Cu" "B.Cu") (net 9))
 (segment (start 114 90.3731) (end 114 58) (width 0.2) (layer "B.Cu") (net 9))
 (segment (start 114 96.1634) (end 119.7903 96.1634) (width 0.2) (layer "B.Cu") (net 9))
 (segment (start 119.7903 96.1634) (end 114 90.3731) (width 0.2) (layer "B.Cu") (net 9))
 (segment (start 119.7903 96.1634) (end 114 96.1634) (width 0.2) (layer "B.Cu") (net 9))
 (segment (start 143.24 99.82) (end 143.24 98.7183) (width 0.2) (layer "B.Cu") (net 4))
 (segment (start 140.9192 96.5792) (end 143.0583 98.7183) (width 0.2) (layer "B.Cu") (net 4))
 (segment (start 140.9192 72.3792) (end 140.9192 96.5792) (width 0.2) (layer "B.Cu") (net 4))
 (segment (start 143.0583 98.7183) (end 143.24 98.7183) (width 0.2) (layer "B.Cu") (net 4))
 (segment (start 133 64.46) (end 140.9192 72.3792) (width 0.2) (layer "B.Cu") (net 4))
 (segment (start 110.755 112.9) (end 114.945 108.71) (width 0.2) (layer "F.Cu") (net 15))
 (segment (start 114.945 108.71) (end 140.8683 108.71) (width 0.2) (layer "F.Cu") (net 15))
 (segment (start 140.8683 108.71) (end 142.1383 107.44) (width 0.2) (layer "F.Cu") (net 15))
 (segment (start 143.24 107.44) (end 142.1383 107.44) (width 0.2) (layer "F.Cu") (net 15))
 (segment (start 193.83 85.25) (end 196.58 82.5) (width 0.2) (layer "F.Cu") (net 5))
 (segment (start 184.6519 85.25) (end 193.83 85.25) (width 0.2) (layer "F.Cu") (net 5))
 (segment (start 175.2335 94.6684) (end 170.225 89.66) (width 0.2) (layer "F.Cu") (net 5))
 (segment (start 175.2335 94.6684) (end 184.6519 85.25) (width 0.2) (layer "F.Cu") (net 5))
 (segment (start 170.225 89.66) (end 143.24 89.66) (width 0.2) (layer "F.Cu") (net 5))
 (segment (start 175.445 94.88) (end 175.2335 94.6684) (width 0.2) (layer "F.Cu") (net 5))
 (segment (start 126 58) (end 152.8689 58) (width 0.2) (layer "F.Cu") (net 12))
 (segment (start 152.8689 58) (end 154.0814 59.2125) (width 0.2) (layer "F.Cu") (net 12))
 (via (at 154.0814 59.2125) (size 0.6) (drill 0.3) (layers "F.Cu" "B.Cu") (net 12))
 (segment (start 162.5 67.6311) (end 162.5 115.5) (width 0.2) (layer "B.Cu") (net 12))
 (segment (start 154.0814 59.2125) (end 162.5 67.6311) (width 0.2) (layer "B.Cu") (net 12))
 (segment (start 186.42 71.5) (end 191.92 77) (width 0.2) (layer "F.Cu") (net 10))
 (segment (start 186.42 71.5) (end 181.1575 76.7625) (width 0.2) (layer "F.Cu") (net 10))
 (segment (start 191.92 77) (end 196.58 77) (width 0.2) (layer "F.Cu") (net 10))
 (segment (start 181.1575 76.7625) (end 112.6242 76.7625) (width 0.2) (layer "F.Cu") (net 10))
 (via (at 112.6242 76.7625) (size 0.6) (drill 0.3) (layers "F.Cu" "B.Cu") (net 10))
 (segment (start 112.4579 97.8394) (end 112.6227 98.0042) (width 0.2) (layer "B.Cu") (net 10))
 (segment (start 112.4579 97.8394) (end 112.6227 98.0042) (width 0.2) (layer "B.Cu") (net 10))
 (segment (start 112.6242 76.7625) (end 112.6242 97.6731) (width 0.2) (layer "B.Cu") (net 10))
 (segment (start 112.6227 108.4923) (end 108.215 112.9) (width 0.2) (layer "B.Cu") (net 10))
 (segment (start 112.6227 98.0042) (end 112.6227 108.4923) (width 0.2) (layer "B.Cu") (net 10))
 (segment (start 112.6242 97.6731) (end 112.4579 97.8394) (width 0.2) (layer "B.Cu") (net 10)))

